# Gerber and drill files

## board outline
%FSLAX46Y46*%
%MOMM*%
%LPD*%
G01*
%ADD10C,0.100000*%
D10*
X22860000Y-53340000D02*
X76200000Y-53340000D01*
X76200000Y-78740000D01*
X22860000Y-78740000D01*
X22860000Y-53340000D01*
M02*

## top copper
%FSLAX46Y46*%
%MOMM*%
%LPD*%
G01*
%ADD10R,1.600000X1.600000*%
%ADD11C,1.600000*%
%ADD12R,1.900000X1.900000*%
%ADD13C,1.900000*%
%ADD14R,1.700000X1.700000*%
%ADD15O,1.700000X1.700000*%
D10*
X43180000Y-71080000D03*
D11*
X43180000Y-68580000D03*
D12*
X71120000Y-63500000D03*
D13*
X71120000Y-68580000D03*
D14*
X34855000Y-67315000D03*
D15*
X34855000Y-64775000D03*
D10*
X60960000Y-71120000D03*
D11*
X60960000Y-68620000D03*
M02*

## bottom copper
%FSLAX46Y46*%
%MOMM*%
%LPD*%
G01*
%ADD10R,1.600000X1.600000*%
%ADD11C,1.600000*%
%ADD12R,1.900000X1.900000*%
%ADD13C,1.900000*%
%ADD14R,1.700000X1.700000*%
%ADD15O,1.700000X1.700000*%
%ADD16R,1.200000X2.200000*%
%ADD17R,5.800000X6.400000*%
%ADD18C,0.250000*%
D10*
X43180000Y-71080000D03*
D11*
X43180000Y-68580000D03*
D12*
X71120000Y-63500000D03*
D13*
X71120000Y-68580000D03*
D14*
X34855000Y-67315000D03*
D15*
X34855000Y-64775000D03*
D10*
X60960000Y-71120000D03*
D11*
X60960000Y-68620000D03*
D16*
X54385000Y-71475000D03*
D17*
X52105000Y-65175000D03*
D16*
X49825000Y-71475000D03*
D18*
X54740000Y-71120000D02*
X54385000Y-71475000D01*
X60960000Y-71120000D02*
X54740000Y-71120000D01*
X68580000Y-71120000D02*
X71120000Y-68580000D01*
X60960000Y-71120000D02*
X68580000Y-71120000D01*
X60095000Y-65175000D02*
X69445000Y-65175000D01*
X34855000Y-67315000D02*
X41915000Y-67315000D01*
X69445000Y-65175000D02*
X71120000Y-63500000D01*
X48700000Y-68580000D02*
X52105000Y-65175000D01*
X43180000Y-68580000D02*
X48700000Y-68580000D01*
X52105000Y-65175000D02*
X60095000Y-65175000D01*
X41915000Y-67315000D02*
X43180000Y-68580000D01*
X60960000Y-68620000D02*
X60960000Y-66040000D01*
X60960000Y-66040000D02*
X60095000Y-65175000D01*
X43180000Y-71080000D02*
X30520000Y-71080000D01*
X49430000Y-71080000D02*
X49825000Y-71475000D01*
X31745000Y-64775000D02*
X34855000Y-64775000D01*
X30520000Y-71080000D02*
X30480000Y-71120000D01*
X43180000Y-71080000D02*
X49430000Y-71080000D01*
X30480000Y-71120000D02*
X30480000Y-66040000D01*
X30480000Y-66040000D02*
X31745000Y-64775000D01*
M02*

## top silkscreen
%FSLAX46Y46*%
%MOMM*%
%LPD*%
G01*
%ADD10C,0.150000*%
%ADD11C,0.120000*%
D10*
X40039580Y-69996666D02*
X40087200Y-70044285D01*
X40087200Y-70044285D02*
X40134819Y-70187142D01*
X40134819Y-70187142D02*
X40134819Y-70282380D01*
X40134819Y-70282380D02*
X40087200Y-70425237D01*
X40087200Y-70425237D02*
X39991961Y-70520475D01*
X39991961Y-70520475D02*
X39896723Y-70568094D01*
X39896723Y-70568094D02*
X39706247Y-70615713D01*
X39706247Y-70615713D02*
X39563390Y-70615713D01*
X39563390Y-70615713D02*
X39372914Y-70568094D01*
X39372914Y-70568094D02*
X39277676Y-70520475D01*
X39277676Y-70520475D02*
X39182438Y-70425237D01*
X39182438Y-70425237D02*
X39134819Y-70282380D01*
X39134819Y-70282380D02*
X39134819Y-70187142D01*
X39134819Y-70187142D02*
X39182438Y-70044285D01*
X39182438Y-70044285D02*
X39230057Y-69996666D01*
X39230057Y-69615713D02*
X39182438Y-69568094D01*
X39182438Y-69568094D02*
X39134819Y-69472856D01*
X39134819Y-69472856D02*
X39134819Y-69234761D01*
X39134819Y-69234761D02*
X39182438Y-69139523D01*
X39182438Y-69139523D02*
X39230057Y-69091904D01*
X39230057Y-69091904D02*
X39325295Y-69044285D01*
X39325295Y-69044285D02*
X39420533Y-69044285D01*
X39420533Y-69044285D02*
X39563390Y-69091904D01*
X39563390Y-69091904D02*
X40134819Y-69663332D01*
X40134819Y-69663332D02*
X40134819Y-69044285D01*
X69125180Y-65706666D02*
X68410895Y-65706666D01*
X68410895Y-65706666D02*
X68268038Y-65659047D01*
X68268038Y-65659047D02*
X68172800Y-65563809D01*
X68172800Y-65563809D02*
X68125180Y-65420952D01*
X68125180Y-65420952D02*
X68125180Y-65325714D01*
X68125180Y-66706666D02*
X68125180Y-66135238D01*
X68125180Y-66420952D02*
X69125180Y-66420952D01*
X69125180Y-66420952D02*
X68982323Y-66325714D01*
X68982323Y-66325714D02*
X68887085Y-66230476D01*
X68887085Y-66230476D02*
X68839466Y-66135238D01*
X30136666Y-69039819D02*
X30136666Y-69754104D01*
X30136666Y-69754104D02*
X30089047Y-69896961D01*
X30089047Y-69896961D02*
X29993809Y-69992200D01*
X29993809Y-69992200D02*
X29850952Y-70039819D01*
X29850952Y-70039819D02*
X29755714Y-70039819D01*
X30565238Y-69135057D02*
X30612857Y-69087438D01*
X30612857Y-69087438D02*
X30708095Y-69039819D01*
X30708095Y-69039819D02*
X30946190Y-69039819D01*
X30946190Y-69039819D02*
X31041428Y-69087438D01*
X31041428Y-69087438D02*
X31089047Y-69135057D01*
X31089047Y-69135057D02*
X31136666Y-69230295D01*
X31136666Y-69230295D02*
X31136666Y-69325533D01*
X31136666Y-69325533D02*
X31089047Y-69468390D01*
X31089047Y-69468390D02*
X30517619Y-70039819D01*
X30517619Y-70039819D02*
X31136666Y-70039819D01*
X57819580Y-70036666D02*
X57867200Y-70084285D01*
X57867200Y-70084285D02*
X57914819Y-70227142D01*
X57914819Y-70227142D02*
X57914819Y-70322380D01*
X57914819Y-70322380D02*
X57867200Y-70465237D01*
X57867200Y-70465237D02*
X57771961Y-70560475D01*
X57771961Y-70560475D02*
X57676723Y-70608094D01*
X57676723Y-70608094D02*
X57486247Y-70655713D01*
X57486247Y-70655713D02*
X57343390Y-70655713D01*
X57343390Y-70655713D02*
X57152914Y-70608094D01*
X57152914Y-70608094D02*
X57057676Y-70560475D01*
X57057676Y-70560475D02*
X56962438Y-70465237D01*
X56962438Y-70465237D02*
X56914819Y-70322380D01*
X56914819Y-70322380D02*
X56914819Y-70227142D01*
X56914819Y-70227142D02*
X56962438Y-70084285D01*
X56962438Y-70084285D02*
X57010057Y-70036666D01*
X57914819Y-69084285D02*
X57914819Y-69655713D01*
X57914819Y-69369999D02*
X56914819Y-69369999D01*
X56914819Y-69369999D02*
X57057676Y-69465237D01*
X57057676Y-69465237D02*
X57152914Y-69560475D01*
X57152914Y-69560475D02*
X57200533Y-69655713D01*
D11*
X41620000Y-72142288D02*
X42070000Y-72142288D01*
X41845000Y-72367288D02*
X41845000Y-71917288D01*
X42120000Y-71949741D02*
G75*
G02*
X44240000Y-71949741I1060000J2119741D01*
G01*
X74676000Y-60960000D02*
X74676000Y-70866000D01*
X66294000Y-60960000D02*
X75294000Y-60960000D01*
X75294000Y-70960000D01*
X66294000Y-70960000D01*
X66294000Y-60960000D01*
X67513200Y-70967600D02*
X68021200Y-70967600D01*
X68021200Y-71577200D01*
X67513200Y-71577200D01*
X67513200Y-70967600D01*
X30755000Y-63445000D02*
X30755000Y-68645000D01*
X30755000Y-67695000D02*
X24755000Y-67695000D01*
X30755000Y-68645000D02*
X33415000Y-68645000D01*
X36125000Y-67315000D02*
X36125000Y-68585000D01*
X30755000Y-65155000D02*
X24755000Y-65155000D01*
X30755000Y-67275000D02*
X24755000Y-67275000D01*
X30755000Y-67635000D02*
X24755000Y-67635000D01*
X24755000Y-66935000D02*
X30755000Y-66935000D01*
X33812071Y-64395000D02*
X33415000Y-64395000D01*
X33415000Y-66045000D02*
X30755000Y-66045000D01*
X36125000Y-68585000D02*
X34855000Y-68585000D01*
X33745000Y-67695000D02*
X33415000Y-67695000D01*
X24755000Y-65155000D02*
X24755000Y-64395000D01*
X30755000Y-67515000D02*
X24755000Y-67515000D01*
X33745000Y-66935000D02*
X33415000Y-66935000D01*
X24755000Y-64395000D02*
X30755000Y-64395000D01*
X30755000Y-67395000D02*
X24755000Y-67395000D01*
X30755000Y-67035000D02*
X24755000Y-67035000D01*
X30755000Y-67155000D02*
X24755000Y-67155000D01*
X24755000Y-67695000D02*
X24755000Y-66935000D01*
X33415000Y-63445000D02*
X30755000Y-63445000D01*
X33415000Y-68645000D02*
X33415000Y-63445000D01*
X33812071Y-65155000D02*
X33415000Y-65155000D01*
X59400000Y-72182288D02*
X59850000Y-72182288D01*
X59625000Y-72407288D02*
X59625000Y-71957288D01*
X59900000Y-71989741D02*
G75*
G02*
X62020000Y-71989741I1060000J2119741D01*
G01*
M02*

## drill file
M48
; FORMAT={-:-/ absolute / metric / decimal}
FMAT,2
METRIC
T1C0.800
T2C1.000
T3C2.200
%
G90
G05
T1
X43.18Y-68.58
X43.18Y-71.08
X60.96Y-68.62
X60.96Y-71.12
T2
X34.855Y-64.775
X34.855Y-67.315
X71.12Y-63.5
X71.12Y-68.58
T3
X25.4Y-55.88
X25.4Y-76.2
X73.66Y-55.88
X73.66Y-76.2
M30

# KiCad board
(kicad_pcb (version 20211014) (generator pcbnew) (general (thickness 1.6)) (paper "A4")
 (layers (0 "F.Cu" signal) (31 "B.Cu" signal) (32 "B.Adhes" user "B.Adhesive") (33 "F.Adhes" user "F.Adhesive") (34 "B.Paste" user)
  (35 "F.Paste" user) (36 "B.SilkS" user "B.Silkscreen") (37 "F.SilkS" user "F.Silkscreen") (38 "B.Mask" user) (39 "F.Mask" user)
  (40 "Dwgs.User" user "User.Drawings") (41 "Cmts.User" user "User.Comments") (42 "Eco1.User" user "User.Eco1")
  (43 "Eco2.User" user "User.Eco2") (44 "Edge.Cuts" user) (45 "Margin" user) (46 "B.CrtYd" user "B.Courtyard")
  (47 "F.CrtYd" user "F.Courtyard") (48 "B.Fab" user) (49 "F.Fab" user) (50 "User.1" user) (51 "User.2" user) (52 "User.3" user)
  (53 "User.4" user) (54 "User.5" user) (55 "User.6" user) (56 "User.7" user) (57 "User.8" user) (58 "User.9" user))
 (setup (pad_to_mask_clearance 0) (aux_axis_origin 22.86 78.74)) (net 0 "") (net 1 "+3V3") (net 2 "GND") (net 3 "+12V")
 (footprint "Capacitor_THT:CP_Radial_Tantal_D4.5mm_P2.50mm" (layer "F.Cu") (at 43.18 71.08 90)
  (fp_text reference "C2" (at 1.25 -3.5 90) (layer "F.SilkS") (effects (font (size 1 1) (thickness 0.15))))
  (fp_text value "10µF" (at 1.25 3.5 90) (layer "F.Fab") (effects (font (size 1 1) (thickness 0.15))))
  (fp_line (start -1.062288 -1.56) (end -1.062288 -1.11) (layer "F.SilkS") (width 0.12))
  (fp_line (start -1.287288 -1.335) (end -0.837288 -1.335) (layer "F.SilkS") (width 0.12))
  (fp_arc (start -0.869741 -1.06) (mid 3.62 0) (end -0.869741 1.06) (layer "F.SilkS") (width 0.12))
  (pad "1" thru_hole rect (at 0 0 90) (size 1.6 1.6) (drill 0.8) (layers *.Cu *.Mask) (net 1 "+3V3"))
  (pad "2" thru_hole circle (at 2.5 0 90) (size 1.6 1.6) (drill 0.8) (layers *.Cu *.Mask) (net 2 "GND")))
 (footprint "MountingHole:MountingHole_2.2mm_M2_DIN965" (layer "F.Cu") (at 25.4 55.88)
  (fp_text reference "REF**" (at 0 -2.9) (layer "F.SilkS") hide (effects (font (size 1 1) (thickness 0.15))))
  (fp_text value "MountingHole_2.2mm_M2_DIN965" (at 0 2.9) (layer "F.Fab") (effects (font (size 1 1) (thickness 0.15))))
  (pad "" np_thru_hole circle (at 0 0) (size 2.2 2.2) (drill 2.2) (layers *.Cu *.Mask)))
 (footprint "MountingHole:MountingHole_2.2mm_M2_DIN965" (layer "F.Cu") (at 73.66 55.88)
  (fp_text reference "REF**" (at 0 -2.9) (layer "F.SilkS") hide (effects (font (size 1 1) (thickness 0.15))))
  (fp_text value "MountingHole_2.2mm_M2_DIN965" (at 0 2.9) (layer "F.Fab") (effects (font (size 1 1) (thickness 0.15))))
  (pad "" np_thru_hole circle (at 0 0) (size 2.2 2.2) (drill 2.2) (layers *.Cu *.Mask)))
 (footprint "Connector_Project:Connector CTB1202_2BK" (layer "F.Cu") (at 71.12 63.5 -90)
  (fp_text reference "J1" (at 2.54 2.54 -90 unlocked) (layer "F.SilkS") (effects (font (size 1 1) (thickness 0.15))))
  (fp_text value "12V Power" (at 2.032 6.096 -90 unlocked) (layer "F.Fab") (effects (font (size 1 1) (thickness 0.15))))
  (fp_line (start -2.54 -3.556) (end 7.366 -3.556) (layer "F.SilkS") (width 0.12))
  (fp_rect (start -2.54 -4.174) (end 7.46 4.826) (layer "F.SilkS") (width 0.12) (fill none))
  (fp_rect (start 7.4676 3.6068) (end 8.0772 3.0988) (layer "F.SilkS") (width 0.12) (fill none))
  (pad "1" thru_hole rect (at 0 0 270) (size 1.9 1.9) (drill 1) (layers *.Cu *.Mask) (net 2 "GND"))
  (pad "2" thru_hole circle (at 5.08 0 270) (size 1.9 1.9) (drill 1) (layers *.Cu *.Mask) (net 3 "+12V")))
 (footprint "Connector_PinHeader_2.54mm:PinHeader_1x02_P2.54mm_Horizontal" (layer "F.Cu") (at 34.855 67.315 180)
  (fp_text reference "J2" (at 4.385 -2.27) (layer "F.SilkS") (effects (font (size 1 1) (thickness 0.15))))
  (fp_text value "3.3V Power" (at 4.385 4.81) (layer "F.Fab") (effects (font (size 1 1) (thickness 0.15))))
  (fp_line (start 4.1 3.87) (end 4.1 -1.33) (layer "F.SilkS") (width 0.12))
  (fp_line (start 4.1 -0.38) (end 10.1 -0.38) (layer "F.SilkS") (width 0.12))
  (fp_line (start 4.1 -1.33) (end 1.44 -1.33) (layer "F.SilkS") (width 0.12))
  (fp_line (start -1.27 0) (end -1.27 -1.27) (layer "F.SilkS") (width 0.12))
  (fp_line (start 4.1 2.16) (end 10.1 2.16) (layer "F.SilkS") (width 0.12))
  (fp_line (start 4.1 0.04) (end 10.1 0.04) (layer "F.SilkS") (width 0.12))
  (fp_line (start 4.1 -0.32) (end 10.1 -0.32) (layer "F.SilkS") (width 0.12))
  (fp_line (start 10.1 0.38) (end 4.1 0.38) (layer "F.SilkS") (width 0.12))
  (fp_line (start 1.042929 2.92) (end 1.44 2.92) (layer "F.SilkS") (width 0.12))
  (fp_line (start 1.44 1.27) (end 4.1 1.27) (layer "F.SilkS") (width 0.12))
  (fp_line (start -1.27 -1.27) (end 0 -1.27) (layer "F.SilkS") (width 0.12))
  (fp_line (start 1.11 -0.38) (end 1.44 -0.38) (layer "F.SilkS") (width 0.12))
  (fp_line (start 10.1 2.16) (end 10.1 2.92) (layer "F.SilkS") (width 0.12))
  (fp_line (start 4.1 -0.2) (end 10.1 -0.2) (layer "F.SilkS") (width 0.12))
  (fp_line (start 1.11 0.38) (end 1.44 0.38) (layer "F.SilkS") (width 0.12))
  (fp_line (start 10.1 2.92) (end 4.1 2.92) (layer "F.SilkS") (width 0.12))
  (fp_line (start 4.1 -0.08) (end 10.1 -0.08) (layer "F.SilkS") (width 0.12))
  (fp_line (start 4.1 0.28) (end 10.1 0.28) (layer "F.SilkS") (width 0.12))
  (fp_line (start 4.1 0.16) (end 10.1 0.16) (layer "F.SilkS") (width 0.12))
  (fp_line (start 10.1 -0.38) (end 10.1 0.38) (layer "F.SilkS") (width 0.12))
  (fp_line (start 1.44 3.87) (end 4.1 3.87) (layer "F.SilkS") (width 0.12))
  (fp_line (start 1.44 -1.33) (end 1.44 3.87) (layer "F.SilkS") (width 0.12))
  (fp_line (start 1.042929 2.16) (end 1.44 2.16) (layer "F.SilkS") (width 0.12))
  (pad "1" thru_hole rect (at 0 0 180) (size 1.7 1.7) (drill 1) (layers *.Cu *.Mask) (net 2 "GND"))
  (pad "2" thru_hole oval (at 0 2.54 180) (size 1.7 1.7) (drill 1) (layers *.Cu *.Mask) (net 1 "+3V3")))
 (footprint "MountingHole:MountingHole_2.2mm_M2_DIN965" (layer "F.Cu") (at 25.4 76.2)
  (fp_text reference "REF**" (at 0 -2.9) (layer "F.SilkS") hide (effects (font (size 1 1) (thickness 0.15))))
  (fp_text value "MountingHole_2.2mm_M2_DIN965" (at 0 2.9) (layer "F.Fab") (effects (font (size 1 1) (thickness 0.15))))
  (pad "" np_thru_hole circle (at 0 0) (size 2.2 2.2) (drill 2.2) (layers *.Cu *.Mask)))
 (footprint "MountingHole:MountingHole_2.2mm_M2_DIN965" (layer "F.Cu") (at 73.66 76.2)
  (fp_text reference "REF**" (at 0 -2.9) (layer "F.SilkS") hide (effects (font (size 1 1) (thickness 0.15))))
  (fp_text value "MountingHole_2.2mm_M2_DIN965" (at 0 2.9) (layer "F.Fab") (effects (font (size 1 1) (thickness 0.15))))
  (pad "" np_thru_hole circle (at 0 0) (size 2.2 2.2) (drill 2.2) (layers *.Cu *.Mask)))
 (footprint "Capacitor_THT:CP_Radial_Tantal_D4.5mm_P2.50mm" (layer "F.Cu") (at 60.96 71.12 90)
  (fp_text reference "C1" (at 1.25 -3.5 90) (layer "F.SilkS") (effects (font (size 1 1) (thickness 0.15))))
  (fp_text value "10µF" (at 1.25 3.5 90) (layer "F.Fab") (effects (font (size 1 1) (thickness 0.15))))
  (fp_line (start -1.062288 -1.56) (end -1.062288 -1.11) (layer "F.SilkS") (width 0.12))
  (fp_line (start -1.287288 -1.335) (end -0.837288 -1.335) (layer "F.SilkS") (width 0.12))
  (fp_arc (start -0.869741 -1.06) (mid 3.62 0) (end -0.869741 1.06) (layer "F.SilkS") (width 0.12))
  (pad "1" thru_hole rect (at 0 0 90) (size 1.6 1.6) (drill 0.8) (layers *.Cu *.Mask) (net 3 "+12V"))
  (pad "2" thru_hole circle (at 2.5 0 90) (size 1.6 1.6) (drill 0.8) (layers *.Cu *.Mask) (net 2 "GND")))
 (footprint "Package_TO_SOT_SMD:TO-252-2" (layer "B.Cu") (at 52.105 67.275 90)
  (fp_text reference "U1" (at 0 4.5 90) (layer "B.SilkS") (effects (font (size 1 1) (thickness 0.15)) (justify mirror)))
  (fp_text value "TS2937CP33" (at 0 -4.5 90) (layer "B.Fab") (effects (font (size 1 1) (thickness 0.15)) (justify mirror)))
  (pad "" smd rect (at 0.425 -1.525 90) (size 3.05 2.75) (layers "B.Paste"))
  (pad "" smd rect (at 0.425 1.525 90) (size 3.05 2.75) (layers "B.Paste"))
  (pad "" smd rect (at 3.775 -1.525 90) (size 3.05 2.75) (layers "B.Paste"))
  (pad "" smd rect (at 3.775 1.525 90) (size 3.05 2.75) (layers "B.Paste"))
  (pad "1" smd rect (at -4.2 2.28 90) (size 2.2 1.2) (layers "B.Cu" "B.Paste" "B.Mask") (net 3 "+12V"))
  (pad "2" smd rect (at 2.1 0 90) (size 6.4 5.8) (layers "B.Cu" "B.Mask") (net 2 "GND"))
  (pad "3" smd rect (at -4.2 -2.28 90) (size 2.2 1.2) (layers "B.Cu" "B.Paste" "B.Mask") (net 1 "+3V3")))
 (gr_rect (start 22.86 53.34) (end 76.2 78.74) (layer "Edge.Cuts") (width 0.1) (fill none))
 (segment (start 54.74 71.12) (end 54.385 71.475) (width 0.25) (layer "B.Cu") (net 3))
 (segment (start 60.96 71.12) (end 54.74 71.12) (width 0.25) (layer "B.Cu") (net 3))
 (segment (start 68.58 71.12) (end 71.12 68.58) (width 0.25) (layer "B.Cu") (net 3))
 (segment (start 60.96 71.12) (end 68.58 71.12) (width 0.25) (layer "B.Cu") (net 3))
 (segment (start 60.095 65.175) (end 69.445 65.175) (width 0.25) (layer "B.Cu") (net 2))
 (segment (start 34.855 67.315) (end 41.915 67.315) (width 0.25) (layer "B.Cu") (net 2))
 (segment (start 69.445 65.175) (end 71.12 63.5) (width 0.25) (layer "B.Cu") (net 2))
 (segment (start 48.7 68.58) (end 52.105 65.175) (width 0.25) (layer "B.Cu") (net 2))
 (segment (start 43.18 68.58) (end 48.7 68.58) (width 0.25) (layer "B.Cu") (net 2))
 (segment (start 52.105 65.175) (end 60.095 65.175) (width 0.25) (layer "B.Cu") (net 2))
 (segment (start 41.915 67.315) (end 43.18 68.58) (width 0.25) (layer "B.Cu") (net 2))
 (segment (start 60.96 68.62) (end 60.96 66.04) (width 0.25) (layer "B.Cu") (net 2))
 (segment (start 60.96 66.04) (end 60.095 65.175) (width 0.25) (layer "B.Cu") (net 2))
 (segment (start 43.18 71.08) (end 30.52 71.08) (width 0.25) (layer "B.Cu") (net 1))
 (segment (start 49.43 71.08) (end 49.825 71.475) (width 0.25) (layer "B.Cu") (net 1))
 (segment (start 31.745 64.775) (end 34.855 64.775) (width 0.25) (layer "B.Cu") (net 1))
 (segment (start 30.52 71.08) (end 30.48 71.12) (width 0.25) (layer "B.Cu") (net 1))
 (segment (start 43.18 71.08) (end 49.43 71.08) (width 0.25) (layer "B.Cu") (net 1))
 (segment (start 30.48 71.12) (end 30.48 66.04) (width 0.25) (layer "B.Cu") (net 1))
 (segment (start 30.48 66.04) (end 31.745 64.775) (width 0.25) (layer "B.Cu") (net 1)))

